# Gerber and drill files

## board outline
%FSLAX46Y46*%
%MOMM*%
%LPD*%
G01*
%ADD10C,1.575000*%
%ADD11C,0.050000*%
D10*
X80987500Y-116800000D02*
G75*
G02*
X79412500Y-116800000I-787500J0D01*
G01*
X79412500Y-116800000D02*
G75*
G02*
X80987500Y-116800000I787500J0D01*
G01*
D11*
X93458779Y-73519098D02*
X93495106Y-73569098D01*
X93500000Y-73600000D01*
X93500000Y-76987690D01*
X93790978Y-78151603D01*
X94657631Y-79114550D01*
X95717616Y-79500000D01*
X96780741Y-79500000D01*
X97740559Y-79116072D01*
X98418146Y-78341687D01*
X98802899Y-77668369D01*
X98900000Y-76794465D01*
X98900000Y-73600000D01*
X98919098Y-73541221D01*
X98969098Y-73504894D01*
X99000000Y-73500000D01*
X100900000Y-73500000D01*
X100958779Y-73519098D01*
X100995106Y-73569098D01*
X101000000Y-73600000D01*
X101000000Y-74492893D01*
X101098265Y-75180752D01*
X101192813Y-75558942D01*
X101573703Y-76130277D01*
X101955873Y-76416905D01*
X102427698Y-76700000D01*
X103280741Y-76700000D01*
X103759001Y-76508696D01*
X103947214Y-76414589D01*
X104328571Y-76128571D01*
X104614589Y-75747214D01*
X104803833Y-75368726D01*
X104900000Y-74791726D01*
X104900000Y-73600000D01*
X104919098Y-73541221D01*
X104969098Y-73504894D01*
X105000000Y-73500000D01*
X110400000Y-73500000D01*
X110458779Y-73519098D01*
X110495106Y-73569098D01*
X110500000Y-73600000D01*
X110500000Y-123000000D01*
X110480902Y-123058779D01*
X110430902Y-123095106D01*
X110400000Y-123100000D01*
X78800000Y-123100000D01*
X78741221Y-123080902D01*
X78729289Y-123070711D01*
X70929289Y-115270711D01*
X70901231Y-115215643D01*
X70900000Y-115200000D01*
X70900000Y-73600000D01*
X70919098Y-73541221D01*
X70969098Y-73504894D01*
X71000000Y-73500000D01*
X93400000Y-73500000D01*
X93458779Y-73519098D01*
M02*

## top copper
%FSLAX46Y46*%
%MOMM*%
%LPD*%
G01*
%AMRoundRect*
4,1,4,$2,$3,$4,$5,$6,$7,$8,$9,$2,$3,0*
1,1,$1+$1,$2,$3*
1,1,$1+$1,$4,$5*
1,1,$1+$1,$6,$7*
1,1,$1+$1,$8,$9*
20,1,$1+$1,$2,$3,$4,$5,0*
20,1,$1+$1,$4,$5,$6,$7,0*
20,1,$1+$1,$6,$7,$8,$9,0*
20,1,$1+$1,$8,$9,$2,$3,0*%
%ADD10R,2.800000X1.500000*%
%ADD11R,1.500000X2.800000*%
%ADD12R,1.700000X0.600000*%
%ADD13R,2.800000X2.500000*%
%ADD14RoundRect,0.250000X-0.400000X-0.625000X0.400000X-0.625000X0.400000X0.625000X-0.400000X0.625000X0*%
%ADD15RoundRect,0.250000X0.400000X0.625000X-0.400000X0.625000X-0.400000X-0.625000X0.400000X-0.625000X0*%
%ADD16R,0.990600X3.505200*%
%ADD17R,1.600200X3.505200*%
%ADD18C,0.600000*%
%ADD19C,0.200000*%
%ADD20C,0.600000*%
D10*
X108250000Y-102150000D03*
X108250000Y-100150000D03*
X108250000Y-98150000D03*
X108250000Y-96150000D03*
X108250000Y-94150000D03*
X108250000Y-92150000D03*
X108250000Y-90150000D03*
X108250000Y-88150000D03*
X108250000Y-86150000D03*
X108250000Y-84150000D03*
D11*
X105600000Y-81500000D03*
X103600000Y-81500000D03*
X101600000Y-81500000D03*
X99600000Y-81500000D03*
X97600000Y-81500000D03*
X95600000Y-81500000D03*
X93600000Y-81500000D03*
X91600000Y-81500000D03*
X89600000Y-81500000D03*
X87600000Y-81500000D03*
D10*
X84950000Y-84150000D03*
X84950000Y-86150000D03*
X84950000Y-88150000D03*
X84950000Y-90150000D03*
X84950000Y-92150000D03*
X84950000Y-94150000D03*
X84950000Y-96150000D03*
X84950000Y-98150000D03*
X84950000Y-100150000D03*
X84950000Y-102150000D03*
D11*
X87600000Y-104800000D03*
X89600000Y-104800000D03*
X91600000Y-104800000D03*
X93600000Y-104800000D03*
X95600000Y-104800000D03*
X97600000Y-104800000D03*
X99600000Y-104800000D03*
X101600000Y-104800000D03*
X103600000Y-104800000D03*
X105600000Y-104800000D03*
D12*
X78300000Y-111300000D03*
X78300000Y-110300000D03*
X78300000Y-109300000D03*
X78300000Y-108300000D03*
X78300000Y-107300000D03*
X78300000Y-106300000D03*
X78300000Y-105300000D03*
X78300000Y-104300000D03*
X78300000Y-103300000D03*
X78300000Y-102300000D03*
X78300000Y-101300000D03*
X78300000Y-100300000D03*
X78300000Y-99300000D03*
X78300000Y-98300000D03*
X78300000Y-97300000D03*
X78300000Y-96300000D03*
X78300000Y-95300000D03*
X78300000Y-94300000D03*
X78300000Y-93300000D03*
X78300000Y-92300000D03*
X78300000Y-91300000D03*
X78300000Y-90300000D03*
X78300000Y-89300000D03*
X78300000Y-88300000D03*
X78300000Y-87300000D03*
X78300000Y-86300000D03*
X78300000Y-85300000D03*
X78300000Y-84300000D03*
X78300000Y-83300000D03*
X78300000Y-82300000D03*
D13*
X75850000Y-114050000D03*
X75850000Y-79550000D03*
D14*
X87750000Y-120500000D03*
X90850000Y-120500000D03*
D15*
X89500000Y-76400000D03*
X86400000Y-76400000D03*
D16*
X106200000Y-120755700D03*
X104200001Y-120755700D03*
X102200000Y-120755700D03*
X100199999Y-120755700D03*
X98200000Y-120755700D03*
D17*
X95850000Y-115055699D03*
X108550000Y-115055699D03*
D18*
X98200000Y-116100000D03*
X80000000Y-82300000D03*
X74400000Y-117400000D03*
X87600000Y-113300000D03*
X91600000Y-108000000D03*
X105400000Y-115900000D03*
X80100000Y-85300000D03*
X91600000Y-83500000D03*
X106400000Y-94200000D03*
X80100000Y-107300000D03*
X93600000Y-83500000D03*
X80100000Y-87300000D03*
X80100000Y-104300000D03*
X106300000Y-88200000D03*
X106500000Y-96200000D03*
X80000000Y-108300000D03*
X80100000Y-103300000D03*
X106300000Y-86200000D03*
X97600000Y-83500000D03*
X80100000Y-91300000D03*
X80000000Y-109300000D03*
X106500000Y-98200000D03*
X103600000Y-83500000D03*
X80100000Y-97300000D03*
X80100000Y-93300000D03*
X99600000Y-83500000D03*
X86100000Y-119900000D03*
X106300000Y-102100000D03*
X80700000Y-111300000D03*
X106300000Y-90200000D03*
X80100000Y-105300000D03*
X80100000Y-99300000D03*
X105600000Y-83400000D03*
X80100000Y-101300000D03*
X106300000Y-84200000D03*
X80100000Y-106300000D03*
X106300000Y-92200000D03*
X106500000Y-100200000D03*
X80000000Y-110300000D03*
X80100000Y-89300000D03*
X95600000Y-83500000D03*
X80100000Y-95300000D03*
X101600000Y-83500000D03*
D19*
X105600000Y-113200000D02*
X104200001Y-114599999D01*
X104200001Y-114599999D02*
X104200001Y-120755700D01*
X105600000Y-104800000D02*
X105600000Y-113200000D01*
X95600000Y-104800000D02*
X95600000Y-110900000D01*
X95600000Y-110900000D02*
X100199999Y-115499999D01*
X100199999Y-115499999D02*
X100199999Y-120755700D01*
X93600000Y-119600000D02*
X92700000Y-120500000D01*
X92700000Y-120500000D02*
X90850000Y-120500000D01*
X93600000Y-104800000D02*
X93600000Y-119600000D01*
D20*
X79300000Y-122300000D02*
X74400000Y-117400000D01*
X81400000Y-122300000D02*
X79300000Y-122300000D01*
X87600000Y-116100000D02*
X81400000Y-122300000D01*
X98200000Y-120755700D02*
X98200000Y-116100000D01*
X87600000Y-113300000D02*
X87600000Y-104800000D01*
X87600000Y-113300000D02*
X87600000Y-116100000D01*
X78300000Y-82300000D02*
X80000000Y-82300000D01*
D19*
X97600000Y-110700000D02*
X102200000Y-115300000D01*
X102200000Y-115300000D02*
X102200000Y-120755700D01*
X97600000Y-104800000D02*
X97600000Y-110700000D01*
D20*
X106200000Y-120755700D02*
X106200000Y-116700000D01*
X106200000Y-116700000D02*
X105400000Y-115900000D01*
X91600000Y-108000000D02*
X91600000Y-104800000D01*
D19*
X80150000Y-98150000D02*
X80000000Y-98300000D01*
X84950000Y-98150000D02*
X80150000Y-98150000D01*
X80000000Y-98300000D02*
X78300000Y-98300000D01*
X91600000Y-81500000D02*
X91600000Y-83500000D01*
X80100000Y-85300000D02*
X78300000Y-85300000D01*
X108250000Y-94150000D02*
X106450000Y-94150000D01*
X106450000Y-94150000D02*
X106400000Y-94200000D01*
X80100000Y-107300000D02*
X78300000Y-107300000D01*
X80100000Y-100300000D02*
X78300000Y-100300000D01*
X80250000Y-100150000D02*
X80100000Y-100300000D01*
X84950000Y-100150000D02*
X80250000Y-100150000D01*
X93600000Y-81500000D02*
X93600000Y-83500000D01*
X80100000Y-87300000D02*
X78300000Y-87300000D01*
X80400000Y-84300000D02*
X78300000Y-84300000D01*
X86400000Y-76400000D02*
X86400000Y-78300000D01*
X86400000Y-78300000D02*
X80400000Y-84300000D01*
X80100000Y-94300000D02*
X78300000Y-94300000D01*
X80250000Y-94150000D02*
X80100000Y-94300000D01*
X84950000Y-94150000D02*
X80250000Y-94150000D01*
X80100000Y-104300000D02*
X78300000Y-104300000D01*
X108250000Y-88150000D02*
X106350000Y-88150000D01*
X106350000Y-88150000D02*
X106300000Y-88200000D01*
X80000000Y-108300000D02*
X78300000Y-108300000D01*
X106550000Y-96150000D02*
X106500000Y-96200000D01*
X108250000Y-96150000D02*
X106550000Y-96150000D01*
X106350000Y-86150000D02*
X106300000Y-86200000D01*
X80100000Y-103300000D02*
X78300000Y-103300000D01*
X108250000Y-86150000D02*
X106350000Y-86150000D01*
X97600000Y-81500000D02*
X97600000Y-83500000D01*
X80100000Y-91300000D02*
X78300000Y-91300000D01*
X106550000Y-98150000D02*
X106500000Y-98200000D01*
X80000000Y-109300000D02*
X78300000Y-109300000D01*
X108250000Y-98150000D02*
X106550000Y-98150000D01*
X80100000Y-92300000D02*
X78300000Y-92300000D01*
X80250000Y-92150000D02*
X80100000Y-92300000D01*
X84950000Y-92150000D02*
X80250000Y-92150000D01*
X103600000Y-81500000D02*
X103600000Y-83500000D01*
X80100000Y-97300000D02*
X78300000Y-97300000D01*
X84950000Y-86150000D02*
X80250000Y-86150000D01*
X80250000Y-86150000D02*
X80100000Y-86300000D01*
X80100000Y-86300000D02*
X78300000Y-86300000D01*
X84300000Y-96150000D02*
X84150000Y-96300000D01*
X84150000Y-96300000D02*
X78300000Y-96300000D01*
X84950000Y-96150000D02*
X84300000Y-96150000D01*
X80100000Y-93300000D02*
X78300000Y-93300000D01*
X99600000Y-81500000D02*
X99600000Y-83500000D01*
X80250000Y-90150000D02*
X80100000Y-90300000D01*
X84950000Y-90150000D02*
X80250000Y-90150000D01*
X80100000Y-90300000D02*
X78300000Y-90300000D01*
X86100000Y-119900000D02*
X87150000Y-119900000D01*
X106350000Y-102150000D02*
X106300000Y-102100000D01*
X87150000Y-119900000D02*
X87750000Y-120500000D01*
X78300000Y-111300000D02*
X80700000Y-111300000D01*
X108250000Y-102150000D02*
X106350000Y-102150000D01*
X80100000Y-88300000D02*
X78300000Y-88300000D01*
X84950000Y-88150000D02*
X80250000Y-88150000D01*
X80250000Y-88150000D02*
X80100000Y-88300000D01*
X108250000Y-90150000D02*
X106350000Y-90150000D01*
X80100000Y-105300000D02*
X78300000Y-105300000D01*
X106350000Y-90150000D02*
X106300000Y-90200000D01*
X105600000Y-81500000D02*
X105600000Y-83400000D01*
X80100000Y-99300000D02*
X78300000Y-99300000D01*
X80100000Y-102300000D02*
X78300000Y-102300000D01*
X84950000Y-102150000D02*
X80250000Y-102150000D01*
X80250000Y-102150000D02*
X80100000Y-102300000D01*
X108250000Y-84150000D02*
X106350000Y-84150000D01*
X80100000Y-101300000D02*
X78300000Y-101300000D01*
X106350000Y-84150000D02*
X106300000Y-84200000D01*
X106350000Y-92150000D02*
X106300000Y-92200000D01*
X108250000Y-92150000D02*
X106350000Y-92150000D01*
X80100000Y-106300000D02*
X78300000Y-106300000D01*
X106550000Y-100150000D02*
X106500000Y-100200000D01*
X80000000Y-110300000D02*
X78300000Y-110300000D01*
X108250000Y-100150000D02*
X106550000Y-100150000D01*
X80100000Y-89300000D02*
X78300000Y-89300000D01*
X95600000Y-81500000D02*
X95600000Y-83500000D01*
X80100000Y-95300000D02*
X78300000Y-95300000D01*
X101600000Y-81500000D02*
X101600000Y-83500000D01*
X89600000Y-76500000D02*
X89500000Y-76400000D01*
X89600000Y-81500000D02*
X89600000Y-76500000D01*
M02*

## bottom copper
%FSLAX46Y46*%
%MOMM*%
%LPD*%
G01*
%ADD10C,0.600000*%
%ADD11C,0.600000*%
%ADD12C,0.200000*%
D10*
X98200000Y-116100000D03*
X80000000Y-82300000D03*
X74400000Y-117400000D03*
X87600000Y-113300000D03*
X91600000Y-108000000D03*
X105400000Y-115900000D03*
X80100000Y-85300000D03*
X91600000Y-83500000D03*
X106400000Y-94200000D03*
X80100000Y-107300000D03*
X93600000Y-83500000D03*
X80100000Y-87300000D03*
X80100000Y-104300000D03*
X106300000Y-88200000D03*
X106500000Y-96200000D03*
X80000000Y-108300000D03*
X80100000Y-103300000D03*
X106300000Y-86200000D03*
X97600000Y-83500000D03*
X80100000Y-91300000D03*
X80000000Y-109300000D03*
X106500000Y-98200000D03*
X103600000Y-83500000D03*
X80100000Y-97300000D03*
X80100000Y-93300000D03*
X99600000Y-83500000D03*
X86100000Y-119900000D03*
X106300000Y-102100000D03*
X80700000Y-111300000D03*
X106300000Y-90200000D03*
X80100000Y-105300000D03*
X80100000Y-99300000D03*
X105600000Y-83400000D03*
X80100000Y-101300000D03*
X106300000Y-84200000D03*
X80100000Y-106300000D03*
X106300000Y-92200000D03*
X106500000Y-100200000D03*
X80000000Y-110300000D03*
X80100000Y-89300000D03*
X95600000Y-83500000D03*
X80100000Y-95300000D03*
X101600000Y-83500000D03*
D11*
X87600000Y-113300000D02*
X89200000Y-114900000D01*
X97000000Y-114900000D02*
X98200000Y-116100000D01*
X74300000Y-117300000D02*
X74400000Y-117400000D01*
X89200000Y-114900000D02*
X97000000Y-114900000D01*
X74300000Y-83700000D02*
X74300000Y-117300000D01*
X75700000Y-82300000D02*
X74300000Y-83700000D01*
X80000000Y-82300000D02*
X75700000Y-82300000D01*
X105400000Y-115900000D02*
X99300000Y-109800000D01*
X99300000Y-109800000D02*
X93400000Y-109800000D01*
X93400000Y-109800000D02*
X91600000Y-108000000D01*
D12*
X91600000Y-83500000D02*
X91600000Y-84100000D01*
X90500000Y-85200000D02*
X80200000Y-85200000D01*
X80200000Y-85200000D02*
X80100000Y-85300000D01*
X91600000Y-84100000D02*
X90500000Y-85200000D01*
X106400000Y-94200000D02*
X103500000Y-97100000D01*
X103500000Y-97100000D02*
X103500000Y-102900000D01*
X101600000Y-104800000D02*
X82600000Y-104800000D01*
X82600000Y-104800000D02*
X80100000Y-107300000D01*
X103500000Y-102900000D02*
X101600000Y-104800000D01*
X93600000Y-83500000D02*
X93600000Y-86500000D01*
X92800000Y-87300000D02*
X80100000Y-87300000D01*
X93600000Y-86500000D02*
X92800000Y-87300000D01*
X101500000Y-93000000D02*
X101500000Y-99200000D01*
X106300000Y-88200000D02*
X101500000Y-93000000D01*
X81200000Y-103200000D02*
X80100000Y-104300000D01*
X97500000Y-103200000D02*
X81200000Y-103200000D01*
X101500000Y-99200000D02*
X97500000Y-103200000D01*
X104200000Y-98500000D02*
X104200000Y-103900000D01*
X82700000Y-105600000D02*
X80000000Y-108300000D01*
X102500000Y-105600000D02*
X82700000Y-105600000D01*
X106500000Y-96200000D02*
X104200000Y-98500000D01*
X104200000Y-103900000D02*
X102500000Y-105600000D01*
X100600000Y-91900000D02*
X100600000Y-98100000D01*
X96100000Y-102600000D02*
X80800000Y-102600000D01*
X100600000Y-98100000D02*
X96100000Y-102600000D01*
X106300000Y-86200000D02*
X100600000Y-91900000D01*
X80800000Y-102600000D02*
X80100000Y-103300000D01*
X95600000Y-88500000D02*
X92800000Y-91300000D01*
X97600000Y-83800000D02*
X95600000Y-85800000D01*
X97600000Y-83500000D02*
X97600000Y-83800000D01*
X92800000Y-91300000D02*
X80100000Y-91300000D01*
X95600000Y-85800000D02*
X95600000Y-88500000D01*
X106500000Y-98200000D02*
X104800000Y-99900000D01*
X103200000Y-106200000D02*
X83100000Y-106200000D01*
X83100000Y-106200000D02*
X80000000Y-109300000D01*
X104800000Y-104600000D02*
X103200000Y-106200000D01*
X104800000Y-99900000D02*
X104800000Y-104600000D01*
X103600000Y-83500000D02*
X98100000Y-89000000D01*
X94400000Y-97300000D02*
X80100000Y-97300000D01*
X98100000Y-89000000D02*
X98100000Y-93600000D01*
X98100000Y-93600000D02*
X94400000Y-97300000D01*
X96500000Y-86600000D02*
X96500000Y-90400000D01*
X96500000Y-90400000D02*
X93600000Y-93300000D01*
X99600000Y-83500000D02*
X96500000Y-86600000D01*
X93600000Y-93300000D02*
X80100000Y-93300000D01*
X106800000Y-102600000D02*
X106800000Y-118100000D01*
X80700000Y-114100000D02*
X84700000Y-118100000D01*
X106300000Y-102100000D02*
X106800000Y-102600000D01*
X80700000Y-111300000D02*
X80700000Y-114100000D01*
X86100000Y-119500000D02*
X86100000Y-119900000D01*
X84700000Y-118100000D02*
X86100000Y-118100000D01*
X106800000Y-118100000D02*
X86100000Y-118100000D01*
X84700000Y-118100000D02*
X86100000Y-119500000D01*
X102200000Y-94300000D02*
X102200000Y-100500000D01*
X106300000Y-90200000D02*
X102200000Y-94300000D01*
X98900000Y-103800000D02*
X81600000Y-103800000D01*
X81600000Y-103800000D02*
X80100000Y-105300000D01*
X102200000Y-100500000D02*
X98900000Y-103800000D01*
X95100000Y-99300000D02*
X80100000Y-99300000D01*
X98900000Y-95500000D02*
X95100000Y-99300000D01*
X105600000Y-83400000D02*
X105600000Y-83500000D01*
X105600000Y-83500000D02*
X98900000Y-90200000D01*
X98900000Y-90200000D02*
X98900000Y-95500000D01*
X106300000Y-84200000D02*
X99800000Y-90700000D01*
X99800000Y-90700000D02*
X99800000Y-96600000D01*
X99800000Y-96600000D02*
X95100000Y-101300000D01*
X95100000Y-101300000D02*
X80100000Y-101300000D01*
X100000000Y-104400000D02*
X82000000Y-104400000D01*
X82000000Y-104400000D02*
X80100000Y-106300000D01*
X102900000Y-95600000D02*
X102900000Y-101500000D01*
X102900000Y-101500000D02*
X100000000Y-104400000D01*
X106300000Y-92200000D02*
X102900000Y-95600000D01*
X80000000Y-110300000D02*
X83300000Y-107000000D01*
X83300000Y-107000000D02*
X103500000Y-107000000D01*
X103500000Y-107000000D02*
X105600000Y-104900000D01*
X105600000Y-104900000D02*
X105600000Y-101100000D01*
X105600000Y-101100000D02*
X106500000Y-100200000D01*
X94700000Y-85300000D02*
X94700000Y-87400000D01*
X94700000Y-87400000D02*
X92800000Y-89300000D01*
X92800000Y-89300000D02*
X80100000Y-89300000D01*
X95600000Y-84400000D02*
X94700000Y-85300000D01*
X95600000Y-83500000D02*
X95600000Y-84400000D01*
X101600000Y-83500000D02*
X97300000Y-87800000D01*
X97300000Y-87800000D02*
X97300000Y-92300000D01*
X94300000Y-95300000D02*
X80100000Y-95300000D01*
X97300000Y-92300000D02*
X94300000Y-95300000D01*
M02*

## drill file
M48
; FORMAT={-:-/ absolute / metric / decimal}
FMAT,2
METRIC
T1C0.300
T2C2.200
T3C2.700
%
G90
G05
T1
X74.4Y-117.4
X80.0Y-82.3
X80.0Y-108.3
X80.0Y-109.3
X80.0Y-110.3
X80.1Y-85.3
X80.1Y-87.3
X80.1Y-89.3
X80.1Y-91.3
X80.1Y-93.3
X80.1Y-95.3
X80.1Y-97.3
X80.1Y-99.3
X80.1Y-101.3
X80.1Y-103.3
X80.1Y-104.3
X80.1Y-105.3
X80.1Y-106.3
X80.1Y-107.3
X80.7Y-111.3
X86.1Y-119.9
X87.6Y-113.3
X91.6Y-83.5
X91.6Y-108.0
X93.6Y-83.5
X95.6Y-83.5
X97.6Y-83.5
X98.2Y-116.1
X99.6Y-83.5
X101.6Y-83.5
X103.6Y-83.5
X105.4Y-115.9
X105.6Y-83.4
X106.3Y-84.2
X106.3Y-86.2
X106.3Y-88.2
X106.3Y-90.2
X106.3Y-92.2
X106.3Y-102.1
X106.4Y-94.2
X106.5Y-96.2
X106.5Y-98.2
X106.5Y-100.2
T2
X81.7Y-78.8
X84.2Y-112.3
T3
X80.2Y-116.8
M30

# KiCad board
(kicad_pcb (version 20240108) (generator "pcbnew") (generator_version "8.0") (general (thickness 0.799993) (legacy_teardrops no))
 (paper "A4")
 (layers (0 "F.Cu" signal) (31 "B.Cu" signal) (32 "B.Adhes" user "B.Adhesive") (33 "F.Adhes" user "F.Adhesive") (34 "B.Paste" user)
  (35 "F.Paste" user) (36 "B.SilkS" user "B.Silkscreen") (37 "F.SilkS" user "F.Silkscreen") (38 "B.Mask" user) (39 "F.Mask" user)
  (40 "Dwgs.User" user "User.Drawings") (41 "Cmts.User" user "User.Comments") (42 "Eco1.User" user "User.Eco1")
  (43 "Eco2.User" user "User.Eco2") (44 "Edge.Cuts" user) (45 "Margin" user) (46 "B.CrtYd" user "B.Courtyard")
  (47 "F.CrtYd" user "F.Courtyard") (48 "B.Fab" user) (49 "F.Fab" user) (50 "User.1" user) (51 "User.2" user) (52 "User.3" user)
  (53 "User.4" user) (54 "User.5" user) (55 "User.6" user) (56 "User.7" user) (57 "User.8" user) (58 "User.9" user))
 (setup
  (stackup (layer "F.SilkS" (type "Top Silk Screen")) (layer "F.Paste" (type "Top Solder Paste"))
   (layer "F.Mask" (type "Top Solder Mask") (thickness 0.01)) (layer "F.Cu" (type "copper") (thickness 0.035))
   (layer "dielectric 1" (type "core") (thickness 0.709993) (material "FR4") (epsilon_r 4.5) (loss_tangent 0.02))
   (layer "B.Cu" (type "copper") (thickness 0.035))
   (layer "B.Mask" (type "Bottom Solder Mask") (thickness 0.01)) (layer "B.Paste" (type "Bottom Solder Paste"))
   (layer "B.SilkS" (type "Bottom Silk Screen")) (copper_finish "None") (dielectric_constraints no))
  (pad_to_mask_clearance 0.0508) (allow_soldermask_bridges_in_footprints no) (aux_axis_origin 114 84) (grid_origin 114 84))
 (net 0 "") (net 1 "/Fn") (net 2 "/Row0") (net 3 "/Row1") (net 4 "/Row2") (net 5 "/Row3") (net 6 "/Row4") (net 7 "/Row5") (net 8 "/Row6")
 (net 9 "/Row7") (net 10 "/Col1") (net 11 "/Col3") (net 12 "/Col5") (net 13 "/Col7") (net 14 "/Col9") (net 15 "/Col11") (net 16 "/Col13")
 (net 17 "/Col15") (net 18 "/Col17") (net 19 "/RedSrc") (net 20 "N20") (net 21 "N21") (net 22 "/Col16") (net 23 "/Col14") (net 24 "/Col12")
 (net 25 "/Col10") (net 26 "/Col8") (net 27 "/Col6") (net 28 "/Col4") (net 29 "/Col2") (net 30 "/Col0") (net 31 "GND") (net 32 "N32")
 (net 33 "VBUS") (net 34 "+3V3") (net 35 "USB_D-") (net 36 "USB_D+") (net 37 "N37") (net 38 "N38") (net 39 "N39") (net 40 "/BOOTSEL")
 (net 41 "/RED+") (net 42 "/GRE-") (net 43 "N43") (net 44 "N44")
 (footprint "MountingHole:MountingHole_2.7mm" (layer "F.Cu") (at 80.2 116.8)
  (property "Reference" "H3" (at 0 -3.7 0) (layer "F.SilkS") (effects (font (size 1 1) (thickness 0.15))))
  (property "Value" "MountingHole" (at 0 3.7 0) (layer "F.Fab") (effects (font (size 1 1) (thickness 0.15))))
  (pad "" np_thru_hole circle (at 0 0) (size 2.7 2.7) (drill 2.7) (layers "*.Cu" "*.Mask")))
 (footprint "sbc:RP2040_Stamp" (layer "F.Cu") (at 96.6 93.15 180)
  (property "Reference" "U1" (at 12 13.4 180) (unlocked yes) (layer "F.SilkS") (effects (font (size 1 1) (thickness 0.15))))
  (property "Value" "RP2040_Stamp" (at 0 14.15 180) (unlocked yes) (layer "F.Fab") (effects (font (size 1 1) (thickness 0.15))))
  (pad "1" smd rect (at -11.65 -9 180) (size 2.8 1.5) (layers "F.Cu" "F.Paste" "F.Mask") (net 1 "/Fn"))
  (pad "2" smd rect (at -11.65 -7 180) (size 2.8 1.5) (layers "F.Cu" "F.Paste" "F.Mask") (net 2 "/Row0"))
  (pad "3" smd rect (at -11.65 -5 180) (size 2.8 1.5) (layers "F.Cu" "F.Paste" "F.Mask") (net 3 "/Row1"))
  (pad "4" smd rect (at -11.65 -3 180) (size 2.8 1.5) (layers "F.Cu" "F.Paste" "F.Mask") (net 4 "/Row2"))
  (pad "5" smd rect (at -11.65 -1 180) (size 2.8 1.5) (layers "F.Cu" "F.Paste" "F.Mask") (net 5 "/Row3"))
  (pad "6" smd rect (at -11.65 1 180) (size 2.8 1.5) (layers "F.Cu" "F.Paste" "F.Mask") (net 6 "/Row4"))
  (pad "7" smd rect (at -11.65 3 180) (size 2.8 1.5) (layers "F.Cu" "F.Paste" "F.Mask") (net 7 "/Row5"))
  (pad "8" smd rect (at -11.65 5 180) (size 2.8 1.5) (layers "F.Cu" "F.Paste" "F.Mask") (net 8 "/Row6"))
  (pad "9" smd rect (at -11.65 7 180) (size 2.8 1.5) (layers "F.Cu" "F.Paste" "F.Mask") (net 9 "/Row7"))
  (pad "10" smd rect (at -11.65 9 180) (size 2.8 1.5) (layers "F.Cu" "F.Paste" "F.Mask") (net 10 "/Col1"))
  (pad "11" smd rect (at -9 11.65 90) (size 2.8 1.5) (layers "F.Cu" "F.Paste" "F.Mask") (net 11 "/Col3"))
  (pad "12" smd rect (at -7 11.65 90) (size 2.8 1.5) (layers "F.Cu" "F.Paste" "F.Mask") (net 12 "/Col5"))
  (pad "13" smd rect (at -5 11.65 90) (size 2.8 1.5) (layers "F.Cu" "F.Paste" "F.Mask") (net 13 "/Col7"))
  (pad "14" smd rect (at -3 11.65 90) (size 2.8 1.5) (layers "F.Cu" "F.Paste" "F.Mask") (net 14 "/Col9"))
  (pad "15" smd rect (at -1 11.65 90) (size 2.8 1.5) (layers "F.Cu" "F.Paste" "F.Mask") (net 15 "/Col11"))
  (pad "16" smd rect (at 1 11.65 90) (size 2.8 1.5) (layers "F.Cu" "F.Paste" "F.Mask") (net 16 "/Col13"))
  (pad "17" smd rect (at 3 11.65 90) (size 2.8 1.5) (layers "F.Cu" "F.Paste" "F.Mask") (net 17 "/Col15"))
  (pad "18" smd rect (at 5 11.65 90) (size 2.8 1.5) (layers "F.Cu" "F.Paste" "F.Mask") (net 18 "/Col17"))
  (pad "19" smd rect (at 7 11.65 90) (size 2.8 1.5) (layers "F.Cu" "F.Paste" "F.Mask") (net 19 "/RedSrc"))
  (pad "20" smd rect (at 9 11.65 90) (size 2.8 1.5) (layers "F.Cu" "F.Paste" "F.Mask") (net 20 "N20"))
  (pad "21" smd rect (at 11.65 9 180) (size 2.8 1.5) (layers "F.Cu" "F.Paste" "F.Mask") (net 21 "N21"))
  (pad "22" smd rect (at 11.65 7 180) (size 2.8 1.5) (layers "F.Cu" "F.Paste" "F.Mask") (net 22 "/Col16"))
  (pad "23" smd rect (at 11.65 5 180) (size 2.8 1.5) (layers "F.Cu" "F.Paste" "F.Mask") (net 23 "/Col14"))
  (pad "24" smd rect (at 11.65 3 180) (size 2.8 1.5) (layers "F.Cu" "F.Paste" "F.Mask") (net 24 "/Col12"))
  (pad "25" smd rect (at 11.65 1 180) (size 2.8 1.5) (layers "F.Cu" "F.Paste" "F.Mask") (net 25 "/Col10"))
  (pad "26" smd rect (at 11.65 -1 180) (size 2.8 1.5) (layers "F.Cu" "F.Paste" "F.Mask") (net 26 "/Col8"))
  (pad "27" smd rect (at 11.65 -3 180) (size 2.8 1.5) (layers "F.Cu" "F.Paste" "F.Mask") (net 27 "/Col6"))
  (pad "28" smd rect (at 11.65 -5 180) (size 2.8 1.5) (layers "F.Cu" "F.Paste" "F.Mask") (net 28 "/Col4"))
  (pad "29" smd rect (at 11.65 -7 180) (size 2.8 1.5) (layers "F.Cu" "F.Paste" "F.Mask") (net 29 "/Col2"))
  (pad "30" smd rect (at 11.65 -9 180) (size 2.8 1.5) (layers "F.Cu" "F.Paste" "F.Mask") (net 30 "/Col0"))
  (pad "31" smd rect (at 9 -11.65 90) (size 2.8 1.5) (layers "F.Cu" "F.Paste" "F.Mask") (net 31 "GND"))
  (pad "32" smd rect (at 7 -11.65 90) (size 2.8 1.5) (layers "F.Cu" "F.Paste" "F.Mask") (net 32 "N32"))
  (pad "33" smd rect (at 5 -11.65 90) (size 2.8 1.5) (layers "F.Cu" "F.Paste" "F.Mask") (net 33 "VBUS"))
  (pad "34" smd rect (at 3 -11.65 90) (size 2.8 1.5) (layers "F.Cu" "F.Paste" "F.Mask") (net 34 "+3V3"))
  (pad "35" smd rect (at 1 -11.65 90) (size 2.8 1.5) (layers "F.Cu" "F.Paste" "F.Mask") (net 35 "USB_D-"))
  (pad "36" smd rect (at -1 -11.65 90) (size 2.8 1.5) (layers "F.Cu" "F.Paste" "F.Mask") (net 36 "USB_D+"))
  (pad "37" smd rect (at -3 -11.65 90) (size 2.8 1.5) (layers "F.Cu" "F.Paste" "F.Mask") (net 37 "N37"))
  (pad "38" smd rect (at -5 -11.65 90) (size 2.8 1.5) (layers "F.Cu" "F.Paste" "F.Mask") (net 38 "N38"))
  (pad "39" smd rect (at -7 -11.65 90) (size 2.8 1.5) (layers "F.Cu" "F.Paste" "F.Mask") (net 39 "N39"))
  (pad "40" smd rect (at -9 -11.65 90) (size 2.8 1.5) (layers "F.Cu" "F.Paste" "F.Mask") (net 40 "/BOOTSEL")))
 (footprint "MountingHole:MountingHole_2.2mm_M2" (layer "F.Cu") (at 81.7 78.8)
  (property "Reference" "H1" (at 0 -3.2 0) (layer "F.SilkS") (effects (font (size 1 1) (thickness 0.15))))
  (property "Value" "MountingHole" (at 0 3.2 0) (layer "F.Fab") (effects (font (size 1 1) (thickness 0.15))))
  (pad "" np_thru_hole circle (at 0 0) (size 2.2 2.2) (drill 2.2) (layers "*.Cu" "*.Mask")))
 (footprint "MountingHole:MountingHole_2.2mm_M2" (layer "F.Cu") (at 84.2 112.3)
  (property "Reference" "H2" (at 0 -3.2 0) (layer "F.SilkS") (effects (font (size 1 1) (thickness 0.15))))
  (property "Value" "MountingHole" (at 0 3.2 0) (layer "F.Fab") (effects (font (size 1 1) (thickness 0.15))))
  (pad "" np_thru_hole circle (at 0 0) (size 2.2 2.2) (drill 2.2) (layers "*.Cu" "*.Mask")))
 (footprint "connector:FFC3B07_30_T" (layer "F.Cu") (at 75.85 96.8 -90)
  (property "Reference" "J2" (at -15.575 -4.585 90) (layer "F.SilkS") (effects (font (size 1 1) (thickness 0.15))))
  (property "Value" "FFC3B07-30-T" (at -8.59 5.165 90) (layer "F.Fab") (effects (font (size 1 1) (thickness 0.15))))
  (pad "1" smd rect (at 14.5 -2.45 270) (size 0.6 1.7) (layers "F.Cu" "F.Paste" "F.Mask") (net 1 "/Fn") (solder_mask_margin 0.102))
  (pad "2" smd rect (at 13.5 -2.45 270) (size 0.6 1.7) (layers "F.Cu" "F.Paste" "F.Mask") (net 2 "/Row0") (solder_mask_margin 0.102))
  (pad "3" smd rect (at 12.5 -2.45 270) (size 0.6 1.7) (layers "F.Cu" "F.Paste" "F.Mask") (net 3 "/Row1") (solder_mask_margin 0.102))
  (pad "4" smd rect (at 11.5 -2.45 270) (size 0.6 1.7) (layers "F.Cu" "F.Paste" "F.Mask") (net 4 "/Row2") (solder_mask_margin 0.102))
  (pad "5" smd rect (at 10.5 -2.45 270) (size 0.6 1.7) (layers "F.Cu" "F.Paste" "F.Mask") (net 5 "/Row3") (solder_mask_margin 0.102))
  (pad "6" smd rect (at 9.5 -2.45 270) (size 0.6 1.7) (layers "F.Cu" "F.Paste" "F.Mask") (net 6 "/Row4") (solder_mask_margin 0.102))
  (pad "7" smd rect (at 8.5 -2.45 270) (size 0.6 1.7) (layers "F.Cu" "F.Paste" "F.Mask") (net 7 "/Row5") (solder_mask_margin 0.102))
  (pad "8" smd rect (at 7.5 -2.45 270) (size 0.6 1.7) (layers "F.Cu" "F.Paste" "F.Mask") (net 8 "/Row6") (solder_mask_margin 0.102))
  (pad "9" smd rect (at 6.5 -2.45 270) (size 0.6 1.7) (layers "F.Cu" "F.Paste" "F.Mask") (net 9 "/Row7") (solder_mask_margin 0.102))
  (pad "10" smd rect (at 5.5 -2.45 270) (size 0.6 1.7) (layers "F.Cu" "F.Paste" "F.Mask") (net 30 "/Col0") (solder_mask_margin 0.102))
  (pad "11" smd rect (at 4.5 -2.45 270) (size 0.6 1.7) (layers "F.Cu" "F.Paste" "F.Mask") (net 10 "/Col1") (solder_mask_margin 0.102))
  (pad "12" smd rect (at 3.5 -2.45 270) (size 0.6 1.7) (layers "F.Cu" "F.Paste" "F.Mask") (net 29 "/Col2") (solder_mask_margin 0.102))
  (pad "13" smd rect (at 2.5 -2.45 270) (size 0.6 1.7) (layers "F.Cu" "F.Paste" "F.Mask") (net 11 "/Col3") (solder_mask_margin 0.102))
  (pad "14" smd rect (at 1.5 -2.45 270) (size 0.6 1.7) (layers "F.Cu" "F.Paste" "F.Mask") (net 28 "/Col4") (solder_mask_margin 0.102))
  (pad "15" smd rect (at 0.5 -2.45 270) (size 0.6 1.7) (layers "F.Cu" "F.Paste" "F.Mask") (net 12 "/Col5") (solder_mask_margin 0.102))
  (pad "16" smd rect (at -0.5 -2.45 270) (size 0.6 1.7) (layers "F.Cu" "F.Paste" "F.Mask") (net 27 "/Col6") (solder_mask_margin 0.102))
  (pad "17" smd rect (at -1.5 -2.45 270) (size 0.6 1.7) (layers "F.Cu" "F.Paste" "F.Mask") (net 13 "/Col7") (solder_mask_margin 0.102))
  (pad "18" smd rect (at -2.5 -2.45 270) (size 0.6 1.7) (layers "F.Cu" "F.Paste" "F.Mask") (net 26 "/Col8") (solder_mask_margin 0.102))
  (pad "19" smd rect (at -3.5 -2.45 270) (size 0.6 1.7) (layers "F.Cu" "F.Paste" "F.Mask") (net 14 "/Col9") (solder_mask_margin 0.102))
  (pad "20" smd rect (at -4.5 -2.45 270) (size 0.6 1.7) (layers "F.Cu" "F.Paste" "F.Mask") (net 25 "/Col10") (solder_mask_margin 0.102))
  (pad "21" smd rect (at -5.5 -2.45 270) (size 0.6 1.7) (layers "F.Cu" "F.Paste" "F.Mask") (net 15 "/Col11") (solder_mask_margin 0.102))
  (pad "22" smd rect (at -6.5 -2.45 270) (size 0.6 1.7) (layers "F.Cu" "F.Paste" "F.Mask") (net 24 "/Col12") (solder_mask_margin 0.102))
  (pad "23" smd rect (at -7.5 -2.45 270) (size 0.6 1.7) (layers "F.Cu" "F.Paste" "F.Mask") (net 16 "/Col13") (solder_mask_margin 0.102))
  (pad "24" smd rect (at -8.5 -2.45 270) (size 0.6 1.7) (layers "F.Cu" "F.Paste" "F.Mask") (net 23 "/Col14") (solder_mask_margin 0.102))
  (pad "25" smd rect (at -9.5 -2.45 270) (size 0.6 1.7) (layers "F.Cu" "F.Paste" "F.Mask") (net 17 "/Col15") (solder_mask_margin 0.102))
  (pad "26" smd rect (at -10.5 -2.45 270) (size 0.6 1.7) (layers "F.Cu" "F.Paste" "F.Mask") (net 22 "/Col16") (solder_mask_margin 0.102))
  (pad "27" smd rect (at -11.5 -2.45 270) (size 0.6 1.7) (layers "F.Cu" "F.Paste" "F.Mask") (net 18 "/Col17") (solder_mask_margin 0.102))
  (pad "28" smd rect (at -12.5 -2.45 270) (size 0.6 1.7) (layers "F.Cu" "F.Paste" "F.Mask") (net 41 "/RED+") (solder_mask_margin 0.102))
  (pad "29" smd rect (at -13.5 -2.45 270) (size 0.6 1.7) (layers "F.Cu" "F.Paste" "F.Mask") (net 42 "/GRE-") (solder_mask_margin 0.102))
  (pad "30" smd rect (at -14.5 -2.45 270) (size 0.6 1.7) (layers "F.Cu" "F.Paste" "F.Mask") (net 31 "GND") (solder_mask_margin 0.102))
  (pad "S1" smd rect (at 17.25 0 270) (size 2.5 2.8) (layers "F.Cu" "F.Paste" "F.Mask") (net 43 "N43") (solder_mask_margin 0.102))
  (pad "S2" smd rect (at -17.25 0 270) (size 2.5 2.8) (layers "F.Cu" "F.Paste" "F.Mask") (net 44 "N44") (solder_mask_margin 0.102)))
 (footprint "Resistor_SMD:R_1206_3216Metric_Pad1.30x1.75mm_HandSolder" (layer "F.Cu") (at 89.3 120.5)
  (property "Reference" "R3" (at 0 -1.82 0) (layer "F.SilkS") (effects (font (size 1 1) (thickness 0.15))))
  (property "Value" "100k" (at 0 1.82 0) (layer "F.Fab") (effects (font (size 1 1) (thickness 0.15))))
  (pad "1" smd roundrect (at -1.55 0) (size 1.3 1.75) (layers "F.Cu" "F.Paste" "F.Mask") (roundrect_rratio 0.192308) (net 1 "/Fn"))
  (pad "2" smd roundrect (at 1.55 0) (size 1.3 1.75) (layers "F.Cu" "F.Paste" "F.Mask") (roundrect_rratio 0.192308) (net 34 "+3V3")))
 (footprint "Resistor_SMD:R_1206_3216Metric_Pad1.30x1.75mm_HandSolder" (layer "F.Cu") (at 87.95 76.4 180)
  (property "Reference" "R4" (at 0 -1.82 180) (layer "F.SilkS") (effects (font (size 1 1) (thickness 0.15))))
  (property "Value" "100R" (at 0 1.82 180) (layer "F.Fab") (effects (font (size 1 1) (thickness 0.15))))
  (pad "1" smd roundrect (at -1.55 0 180) (size 1.3 1.75) (layers "F.Cu" "F.Paste" "F.Mask") (roundrect_rratio 0.192308) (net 19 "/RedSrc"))
  (pad "2" smd roundrect (at 1.55 0 180) (size 1.3 1.75) (layers "F.Cu" "F.Paste" "F.Mask") (roundrect_rratio 0.192308) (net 41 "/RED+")))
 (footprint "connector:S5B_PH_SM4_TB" (layer "F.Cu") (at 102.2 117.3)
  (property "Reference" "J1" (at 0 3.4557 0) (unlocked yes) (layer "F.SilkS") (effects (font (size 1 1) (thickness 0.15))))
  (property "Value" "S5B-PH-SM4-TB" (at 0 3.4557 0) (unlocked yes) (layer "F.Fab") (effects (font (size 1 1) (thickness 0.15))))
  (pad "1" smd rect (at 4 3.4557) (size 0.9906 3.5052) (layers "F.Cu" "F.Paste" "F.Mask") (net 33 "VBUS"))
  (pad "2" smd rect (at 2.000001 3.4557) (size 0.9906 3.5052) (layers "F.Cu" "F.Paste" "F.Mask") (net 40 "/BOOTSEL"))
  (pad "3" smd rect (at 0 3.4557) (size 0.9906 3.5052) (layers "F.Cu" "F.Paste" "F.Mask") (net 36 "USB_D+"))
  (pad "4" smd rect (at -2.000001 3.4557) (size 0.9906 3.5052) (layers "F.Cu" "F.Paste" "F.Mask") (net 35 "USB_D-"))
  (pad "5" smd rect (at -4 3.4557) (size 0.9906 3.5052) (layers "F.Cu" "F.Paste" "F.Mask") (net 31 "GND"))
  (pad "6" smd rect (at -6.35 -2.244301) (size 1.6002 3.5052) (layers "F.Cu" "F.Paste" "F.Mask"))
  (pad "7" smd rect (at 6.35 -2.244301) (size 1.6002 3.5052) (layers "F.Cu" "F.Paste" "F.Mask")))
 (gr_circle (center 80.2 116.8) (end 81.75 116.8) (stroke (width 0.05) (type solid)) (fill solid) (layer "Edge.Cuts"))
 (gr_poly
  (pts (xy 93.458779 73.519098) (xy 93.495106 73.569098) (xy 93.5 73.6) (xy 93.5 76.98769) (xy 93.790978 78.151603) (xy 94.657631 79.11455)
   (xy 95.717616 79.5) (xy 96.780741 79.5) (xy 97.740559 79.116072) (xy 98.418146 78.341687) (xy 98.802899 77.668369) (xy 98.9 76.794465)
   (xy 98.9 73.6) (xy 98.919098 73.541221) (xy 98.969098 73.504894) (xy 99 73.5) (xy 100.9 73.5) (xy 100.958779 73.519098)
   (xy 100.995106 73.569098) (xy 101 73.6) (xy 101 74.492893) (xy 101.098265 75.180752) (xy 101.192813 75.558942) (xy 101.573703 76.130277)
   (xy 101.955873 76.416905) (xy 102.427698 76.7) (xy 103.280741 76.7) (xy 103.759001 76.508696) (xy 103.947214 76.414589)
   (xy 104.328571 76.128571) (xy 104.614589 75.747214) (xy 104.803833 75.368726) (xy 104.9 74.791726) (xy 104.9 73.6)
   (xy 104.919098 73.541221) (xy 104.969098 73.504894) (xy 105 73.5) (xy 110.4 73.5) (xy 110.458779 73.519098) (xy 110.495106 73.569098)
   (xy 110.5 73.6) (xy 110.5 123) (xy 110.480902 123.058779) (xy 110.430902 123.095106) (xy 110.4 123.1) (xy 78.8 123.1)
   (xy 78.741221 123.080902) (xy 78.729289 123.070711) (xy 70.929289 115.270711) (xy 70.901231 115.215643) (xy 70.9 115.2) (xy 70.9 73.6)
   (xy 70.919098 73.541221) (xy 70.969098 73.504894) (xy 71 73.5) (xy 93.4 73.5))
  (stroke (width 0.05) (type solid)) (fill none) (layer "Edge.Cuts"))
 (segment (start 105.6 113.2) (end 104.200001 114.599999) (width 0.2) (layer "F.Cu") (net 40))
 (segment (start 104.200001 114.599999) (end 104.200001 120.7557) (width 0.2) (layer "F.Cu") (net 40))
 (segment (start 105.6 104.8) (end 105.6 113.2) (width 0.2) (layer "F.Cu") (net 40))
 (segment (start 95.6 104.8) (end 95.6 110.9) (width 0.2) (layer "F.Cu") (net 35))
 (segment (start 95.6 110.9) (end 100.199999 115.499999) (width 0.2) (layer "F.Cu") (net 35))
 (segment (start 100.199999 115.499999) (end 100.199999 120.7557) (width 0.2) (layer "F.Cu") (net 35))
 (segment (start 93.6 119.6) (end 92.7 120.5) (width 0.2) (layer "F.Cu") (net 34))
 (segment (start 92.7 120.5) (end 90.85 120.5) (width 0.2) (layer "F.Cu") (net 34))
 (segment (start 93.6 104.8) (end 93.6 119.6) (width 0.2) (layer "F.Cu") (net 34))
 (segment (start 79.3 122.3) (end 74.4 117.4) (width 0.6) (layer "F.Cu") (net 31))
 (segment (start 81.4 122.3) (end 79.3 122.3) (width 0.6) (layer "F.Cu") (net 31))
 (segment (start 87.6 116.1) (end 81.4 122.3) (width 0.6) (layer "F.Cu") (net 31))
 (segment (start 98.2 120.7557) (end 98.2 116.1) (width 0.6) (layer "F.Cu") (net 31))
 (segment (start 87.6 113.3) (end 87.6 104.8) (width 0.6) (layer "F.Cu") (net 31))
 (segment (start 87.6 113.3) (end 87.6 116.1) (width 0.6) (layer "F.Cu") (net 31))
 (segment (start 78.3 82.3) (end 80 82.3) (width 0.6) (layer "F.Cu") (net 31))
 (via (at 98.2 116.1) (size 0.6) (drill 0.3) (layers "F.Cu" "B.Cu") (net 31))
 (via (at 80 82.3) (size 0.6) (drill 0.3) (layers "F.Cu" "B.Cu") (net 31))
 (via (at 74.4 117.4) (size 0.6) (drill 0.3) (layers "F.Cu" "B.Cu") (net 31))
 (via (at 87.6 113.3) (size 0.6) (drill 0.3) (layers "F.Cu" "B.Cu") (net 31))
 (segment (start 87.6 113.3) (end 89.2 114.9) (width 0.6) (layer "B.Cu") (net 31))
 (segment (start 97 114.9) (end 98.2 116.1) (width 0.6) (layer "B.Cu") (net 31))
 (segment (start 74.3 117.3) (end 74.4 117.4) (width 0.6) (layer "B.Cu") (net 31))
 (segment (start 89.2 114.9) (end 97 114.9) (width 0.6) (layer "B.Cu") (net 31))
 (segment (start 74.3 83.7) (end 74.3 117.3) (width 0.6) (layer "B.Cu") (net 31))
 (segment (start 75.7 82.3) (end 74.3 83.7) (width 0.6) (layer "B.Cu") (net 31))
 (segment (start 80 82.3) (end 75.7 82.3) (width 0.6) (layer "B.Cu") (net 31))
 (segment (start 97.6 110.7) (end 102.2 115.3) (width 0.2) (layer "F.Cu") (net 36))
 (segment (start 102.2 115.3) (end 102.2 120.7557) (width 0.2) (layer "F.Cu") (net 36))
 (segment (start 97.6 104.8) (end 97.6 110.7) (width 0.2) (layer "F.Cu") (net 36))
 (segment (start 106.2 120.7557) (end 106.2 116.7) (width 0.6) (layer "F.Cu") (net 33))
 (segment (start 106.2 116.7) (end 105.4 115.9) (width 0.6) (layer "F.Cu") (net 33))
 (segment (start 91.6 108) (end 91.6 104.8) (width 0.6) (layer "F.Cu") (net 33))
 (via (at 91.6 108) (size 0.6) (drill 0.3) (layers "F.Cu" "B.Cu") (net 33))
 (via (at 105.4 115.9) (size 0.6) (drill 0.3) (layers "F.Cu" "B.Cu") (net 33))
 (segment (start 105.4 115.9) (end 99.3 109.8) (width 0.6) (layer "B.Cu") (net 33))
 (segment (start 99.3 109.8) (end 93.4 109.8) (width 0.6) (layer "B.Cu") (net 33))
 (segment (start 93.4 109.8) (end 91.6 108) (width 0.6) (layer "B.Cu") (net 33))
 (segment (start 80.15 98.15) (end 80 98.3) (width 0.2) (layer "F.Cu") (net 28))
 (segment (start 84.95 98.15) (end 80.15 98.15) (width 0.2) (layer "F.Cu") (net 28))
 (segment (start 80 98.3) (end 78.3 98.3) (width 0.2) (layer "F.Cu") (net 28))
 (segment (start 91.6 81.5) (end 91.6 83.5) (width 0.2) (layer "F.Cu") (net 18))
 (segment (start 80.1 85.3) (end 78.3 85.3) (width 0.2) (layer "F.Cu") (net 18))
 (via (at 80.1 85.3) (size 0.6) (drill 0.3) (layers "F.Cu" "B.Cu") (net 18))
 (via (at 91.6 83.5) (size 0.6) (drill 0.3) (layers "F.Cu" "B.Cu") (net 18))
 (segment (start 91.6 83.5) (end 91.6 84.1) (width 0.2) (layer "B.Cu") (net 18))
 (segment (start 90.5 85.2) (end 80.2 85.2) (width 0.2) (layer "B.Cu") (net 18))
 (segment (start 80.2 85.2) (end 80.1 85.3) (width 0.2) (layer "B.Cu") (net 18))
 (segment (start 91.6 84.1) (end 90.5 85.2) (width 0.2) (layer "B.Cu") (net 18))
 (segment (start 108.25 94.15) (end 106.45 94.15) (width 0.2) (layer "F.Cu") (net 5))
 (segment (start 106.45 94.15) (end 106.4 94.2) (width 0.2) (layer "F.Cu") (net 5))
 (segment (start 80.1 107.3) (end 78.3 107.3) (width 0.2) (layer "F.Cu") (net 5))
 (via (at 106.4 94.2) (size 0.6) (drill 0.3) (layers "F.Cu" "B.Cu") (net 5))
 (via (at 80.1 107.3) (size 0.6) (drill 0.3) (layers "F.Cu" "B.Cu") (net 5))
 (segment (start 106.4 94.2) (end 103.5 97.1) (width 0.2) (layer "B.Cu") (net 5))
 (segment (start 103.5 97.1) (end 103.5 102.9) (width 0.2) (layer "B.Cu") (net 5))
 (segment (start 101.6 104.8) (end 82.6 104.8) (width 0.2) (layer "B.Cu") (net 5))
 (segment (start 82.6 104.8) (end 80.1 107.3) (width 0.2) (layer "B.Cu") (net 5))
 (segment (start 103.5 102.9) (end 101.6 104.8) (width 0.2) (layer "B.Cu") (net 5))
 (segment (start 80.1 100.3) (end 78.3 100.3) (width 0.2) (layer "F.Cu") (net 29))
 (segment (start 80.25 100.15) (end 80.1 100.3) (width 0.2) (layer "F.Cu") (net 29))
 (segment (start 84.95 100.15) (end 80.25 100.15) (width 0.2) (layer "F.Cu") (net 29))
 (segment (start 93.6 81.5) (end 93.6 83.5) (width 0.2) (layer "F.Cu") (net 17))
 (segment (start 80.1 87.3) (end 78.3 87.3) (width 0.2) (layer "F.Cu") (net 17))
 (via (at 93.6 83.5) (size 0.6) (drill 0.3) (layers "F.Cu" "B.Cu") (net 17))
 (via (at 80.1 87.3) (size 0.6) (drill 0.3) (layers "F.Cu" "B.Cu") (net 17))
 (segment (start 93.6 83.5) (end 93.6 86.5) (width 0.2) (layer "B.Cu") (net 17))
 (segment (start 92.8 87.3) (end 80.1 87.3) (width 0.2) (layer "B.Cu") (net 17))
 (segment (start 93.6 86.5) (end 92.8 87.3) (width 0.2) (layer "B.Cu") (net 17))
 (segment (start 80.4 84.3) (end 78.3 84.3) (width 0.2) (layer "F.Cu") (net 41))
 (segment (start 86.4 76.4) (end 86.4 78.3) (width 0.2) (layer "F.Cu") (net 41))
 (segment (start 86.4 78.3) (end 80.4 84.3) (width 0.2) (layer "F.Cu") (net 41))
 (segment (start 80.1 94.3) (end 78.3 94.3) (width 0.2) (layer "F.Cu") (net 26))
 (segment (start 80.25 94.15) (end 80.1 94.3) (width 0.2) (layer "F.Cu") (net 26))
 (segment (start 84.95 94.15) (end 80.25 94.15) (width 0.2) (layer "F.Cu") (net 26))
 (segment (start 80.1 104.3) (end 78.3 104.3) (width 0.2) (layer "F.Cu") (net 8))
 (segment (start 108.25 88.15) (end 106.35 88.15) (width 0.2) (layer "F.Cu") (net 8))
 (segment (start 106.35 88.15) (end 106.3 88.2) (width 0.2) (layer "F.Cu") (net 8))
 (via (at 80.1 104.3) (size 0.6) (drill 0.3) (layers "F.Cu" "B.Cu") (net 8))
 (via (at 106.3 88.2) (size 0.6) (drill 0.3) (layers "F.Cu" "B.Cu") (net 8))
 (segment (start 101.5 93) (end 101.5 99.2) (width 0.2) (layer "B.Cu") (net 8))
 (segment (start 106.3 88.2) (end 101.5 93) (width 0.2) (layer "B.Cu") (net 8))
 (segment (start 81.2 103.2) (end 80.1 104.3) (width 0.2) (layer "B.Cu") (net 8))
 (segment (start 97.5 103.2) (end 81.2 103.2) (width 0.2) (layer "B.Cu") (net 8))
 (segment (start 101.5 99.2) (end 97.5 103.2) (width 0.2) (layer "B.Cu") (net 8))
 (segment (start 80 108.3) (end 78.3 108.3) (width 0.2) (layer "F.Cu") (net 4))
 (segment (start 106.55 96.15) (end 106.5 96.2) (width 0.2) (layer "F.Cu") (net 4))
 (segment (start 108.25 96.15) (end 106.55 96.15) (width 0.2) (layer "F.Cu") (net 4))
 (via (at 106.5 96.2) (size 0.6) (drill 0.3) (layers "F.Cu" "B.Cu") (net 4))
 (via (at 80 108.3) (size 0.6) (drill 0.3) (layers "F.Cu" "B.Cu") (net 4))
 (segment (start 104.2 98.5) (end 104.2 103.9) (width 0.2) (layer "B.Cu") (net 4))
 (segment (start 82.7 105.6) (end 80 108.3) (width 0.2) (layer "B.Cu") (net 4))
 (segment (start 102.5 105.6) (end 82.7 105.6) (width 0.2) (layer "B.Cu") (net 4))
 (segment (start 106.5 96.2) (end 104.2 98.5) (width 0.2) (layer "B.Cu") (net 4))
 (segment (start 104.2 103.9) (end 102.5 105.6) (width 0.2) (layer "B.Cu") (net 4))
 (segment (start 106.35 86.15) (end 106.3 86.2) (width 0.2) (layer "F.Cu") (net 9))
 (segment (start 80.1 103.3) (end 78.3 103.3) (width 0.2) (layer "F.Cu") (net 9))
 (segment (start 108.25 86.15) (end 106.35 86.15) (width 0.2) (layer "F.Cu") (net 9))
 (via (at 80.1 103.3) (size 0.6) (drill 0.3) (layers "F.Cu" "B.Cu") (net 9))
 (via (at 106.3 86.2) (size 0.6) (drill 0.3) (layers "F.Cu" "B.Cu") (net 9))
 (segment (start 100.6 91.9) (end 100.6 98.1) (width 0.2) (layer "B.Cu") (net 9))
 (segment (start 96.1 102.6) (end 80.8 102.6) (width 0.2) (layer "B.Cu") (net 9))
 (segment (start 100.6 98.1) (end 96.1 102.6) (width 0.2) (layer "B.Cu") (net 9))
 (segment (start 106.3 86.2) (end 100.6 91.9) (width 0.2) (layer "B.Cu") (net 9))
 (segment (start 80.8 102.6) (end 80.1 103.3) (width 0.2) (layer "B.Cu") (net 9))
 (segment (start 97.6 81.5) (end 97.6 83.5) (width 0.2) (layer "F.Cu") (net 15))
 (segment (start 80.1 91.3) (end 78.3 91.3) (width 0.2) (layer "F.Cu") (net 15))
 (via (at 97.6 83.5) (size 0.6) (drill 0.3) (layers "F.Cu" "B.Cu") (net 15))
 (via (at 80.1 91.3) (size 0.6) (drill 0.3) (layers "F.Cu" "B.Cu") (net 15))
 (segment (start 95.6 88.5) (end 92.8 91.3) (width 0.2) (layer "B.Cu") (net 15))
 (segment (start 97.6 83.8) (end 95.6 85.8) (width 0.2) (layer "B.Cu") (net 15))
 (segment (start 97.6 83.5) (end 97.6 83.8) (width 0.2) (layer "B.Cu") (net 15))
 (segment (start 92.8 91.3) (end 80.1 91.3) (width 0.2) (layer "B.Cu") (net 15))
 (segment (start 95.6 85.8) (end 95.6 88.5) (width 0.2) (layer "B.Cu") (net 15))
 (segment (start 106.55 98.15) (end 106.5 98.2) (width 0.2) (layer "F.Cu") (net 3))
 (segment (start 80 109.3) (end 78.3 109.3) (width 0.2) (layer "F.Cu") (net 3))
 (segment (start 108.25 98.15) (end 106.55 98.15) (width 0.2) (layer "F.Cu") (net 3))
 (via (at 80 109.3) (size 0.6) (drill 0.3) (layers "F.Cu" "B.Cu") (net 3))
 (via (at 106.5 98.2) (size 0.6) (drill 0.3) (layers "F.Cu" "B.Cu") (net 3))
 (segment (start 106.5 98.2) (end 104.8 99.9) (width 0.2) (layer "B.Cu") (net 3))
 (segment (start 103.2 106.2) (end 83.1 106.2) (width 0.2) (layer "B.Cu") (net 3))
 (segment (start 83.1 106.2) (end 80 109.3) (width 0.2) (layer "B.Cu") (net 3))
 (segment (start 104.8 104.6) (end 103.2 106.2) (width 0.2) (layer "B.Cu") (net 3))
 (segment (start 104.8 99.9) (end 104.8 104.6) (width 0.2) (layer "B.Cu") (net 3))
 (segment (start 80.1 92.3) (end 78.3 92.3) (width 0.2) (layer "F.Cu") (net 25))
 (segment (start 80.25 92.15) (end 80.1 92.3) (width 0.2) (layer "F.Cu") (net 25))
 (segment (start 84.95 92.15) (end 80.25 92.15) (width 0.2) (layer "F.Cu") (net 25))
 (segment (start 103.6 81.5) (end 103.6 83.5) (width 0.2) (layer "F.Cu") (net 12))
 (segment (start 80.1 97.3) (end 78.3 97.3) (width 0.2) (layer "F.Cu") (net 12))
 (via (at 103.6 83.5) (size 0.6) (drill 0.3) (layers "F.Cu" "B.Cu") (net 12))
 (via (at 80.1 97.3) (size 0.6) (drill 0.3) (layers "F.Cu" "B.Cu") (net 12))
 (segment (start 103.6 83.5) (end 98.1 89) (width 0.2) (layer "B.Cu") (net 12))
 (segment (start 94.4 97.3) (end 80.1 97.3) (width 0.2) (layer "B.Cu") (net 12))
 (segment (start 98.1 89) (end 98.1 93.6) (width 0.2) (layer "B.Cu") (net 12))
 (segment (start 98.1 93.6) (end 94.4 97.3) (width 0.2) (layer "B.Cu") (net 12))
 (segment (start 84.95 86.15) (end 80.25 86.15) (width 0.2) (layer "F.Cu") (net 22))
 (segment (start 80.25 86.15) (end 80.1 86.3) (width 0.2) (layer "F.Cu") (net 22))
 (segment (start 80.1 86.3) (end 78.3 86.3) (width 0.2) (layer "F.Cu") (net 22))
 (segment (start 84.3 96.15) (end 84.15 96.3) (width 0.2) (layer "F.Cu") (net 27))
 (segment (start 84.15 96.3) (end 78.3 96.3) (width 0.2) (layer "F.Cu") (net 27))
 (segment (start 84.95 96.15) (end 84.3 96.15) (width 0.2) (layer "F.Cu") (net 27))
 (segment (start 80.1 93.3) (end 78.3 93.3) (width 0.2) (layer "F.Cu") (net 14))
 (segment (start 99.6 81.5) (end 99.6 83.5) (width 0.2) (layer "F.Cu") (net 14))
 (via (at 80.1 93.3) (size 0.6) (drill 0.3) (layers "F.Cu" "B.Cu") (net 14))
 (via (at 99.6 83.5) (size 0.6) (drill 0.3) (layers "F.Cu" "B.Cu") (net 14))
 (segment (start 96.5 86.6) (end 96.5 90.4) (width 0.2) (layer "B.Cu") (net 14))
 (segment (start 96.5 90.4) (end 93.6 93.3) (width 0.2) (layer "B.Cu") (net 14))
 (segment (start 99.6 83.5) (end 96.5 86.6) (width 0.2) (layer "B.Cu") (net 14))
 (segment (start 93.6 93.3) (end 80.1 93.3) (width 0.2) (layer "B.Cu") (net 14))
 (segment (start 80.25 90.15) (end 80.1 90.3) (width 0.2) (layer "F.Cu") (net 24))
 (segment (start 84.95 90.15) (end 80.25 90.15) (width 0.2) (layer "F.Cu") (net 24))
 (segment (start 80.1 90.3) (end 78.3 90.3) (width 0.2) (layer "F.Cu") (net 24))
 (segment (start 86.1 119.9) (end 87.15 119.9) (width 0.2) (layer "F.Cu") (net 1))
 (segment (start 106.35 102.15) (end 106.3 102.1) (width 0.2) (layer "F.Cu") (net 1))
 (segment (start 87.15 119.9) (end 87.75 120.5) (width 0.2) (layer "F.Cu") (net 1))
 (segment (start 78.3 111.3) (end 80.7 111.3) (width 0.2) (layer "F.Cu") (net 1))
 (segment (start 108.25 102.15) (end 106.35 102.15) (width 0.2) (layer "F.Cu") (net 1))
 (via (at 86.1 119.9) (size 0.6) (drill 0.3) (layers "F.Cu" "B.Cu") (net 1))
 (via (at 106.3 102.1) (size 0.6) (drill 0.3) (layers "F.Cu" "B.Cu") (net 1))
 (via (at 80.7 111.3) (size 0.6) (drill 0.3) (layers "F.Cu" "B.Cu") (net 1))
 (segment (start 106.8 102.6) (end 106.8 118.1) (width 0.2) (layer "B.Cu") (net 1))
 (segment (start 80.7 114.1) (end 84.7 118.1) (width 0.2) (layer "B.Cu") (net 1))
 (segment (start 106.3 102.1) (end 106.8 102.6) (width 0.2) (layer "B.Cu") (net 1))
 (segment (start 80.7 111.3) (end 80.7 114.1) (width 0.2) (layer "B.Cu") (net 1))
 (segment (start 86.1 119.5) (end 86.1 119.9) (width 0.2) (layer "B.Cu") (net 1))
 (segment (start 84.7 118.1) (end 86.1 118.1) (width 0.2) (layer "B.Cu") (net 1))
 (segment (start 106.8 118.1) (end 86.1 118.1) (width 0.2) (layer "B.Cu") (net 1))
 (segment (start 84.7 118.1) (end 86.1 119.5) (width 0.2) (layer "B.Cu") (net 1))
 (segment (start 80.1 88.3) (end 78.3 88.3) (width 0.2) (layer "F.Cu") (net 23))
 (segment (start 84.95 88.15) (end 80.25 88.15) (width 0.2) (layer "F.Cu") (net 23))
 (segment (start 80.25 88.15) (end 80.1 88.3) (width 0.2) (layer "F.Cu") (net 23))
 (segment (start 108.25 90.15) (end 106.35 90.15) (width 0.2) (layer "F.Cu") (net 7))
 (segment (start 80.1 105.3) (end 78.3 105.3) (width 0.2) (layer "F.Cu") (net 7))
 (segment (start 106.35 90.15) (end 106.3 90.2) (width 0.2) (layer "F.Cu") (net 7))
 (via (at 106.3 90.2) (size 0.6) (drill 0.3) (layers "F.Cu" "B.Cu") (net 7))
 (via (at 80.1 105.3) (size 0.6) (drill 0.3) (layers "F.Cu" "B.Cu") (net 7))
 (segment (start 102.2 94.3) (end 102.2 100.5) (width 0.2) (layer "B.Cu") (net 7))
 (segment (start 106.3 90.2) (end 102.2 94.3) (width 0.2) (layer "B.Cu") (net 7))
 (segment (start 98.9 103.8) (end 81.6 103.8) (width 0.2) (layer "B.Cu") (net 7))
 (segment (start 81.6 103.8) (end 80.1 105.3) (width 0.2) (layer "B.Cu") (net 7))
 (segment (start 102.2 100.5) (end 98.9 103.8) (width 0.2) (layer "B.Cu") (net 7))
 (segment (start 105.6 81.5) (end 105.6 83.4) (width 0.2) (layer "F.Cu") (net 11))
 (segment (start 80.1 99.3) (end 78.3 99.3) (width 0.2) (layer "F.Cu") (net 11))
 (via (at 80.1 99.3) (size 0.6) (drill 0.3) (layers "F.Cu" "B.Cu") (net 11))
 (via (at 105.6 83.4) (size 0.6) (drill 0.3) (layers "F.Cu" "B.Cu") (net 11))
 (segment (start 95.1 99.3) (end 80.1 99.3) (width 0.2) (layer "B.Cu") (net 11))
 (segment (start 98.9 95.5) (end 95.1 99.3) (width 0.2) (layer "B.Cu") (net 11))
 (segment (start 105.6 83.4) (end 105.6 83.5) (width 0.2) (layer "B.Cu") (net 11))
 (segment (start 105.6 83.5) (end 98.9 90.2) (width 0.2) (layer "B.Cu") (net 11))
 (segment (start 98.9 90.2) (end 98.9 95.5) (width 0.2) (layer "B.Cu") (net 11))
 (segment (start 80.1 102.3) (end 78.3 102.3) (width 0.2) (layer "F.Cu") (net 30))
 (segment (start 84.95 102.15) (end 80.25 102.15) (width 0.2) (layer "F.Cu") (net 30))
 (segment (start 80.25 102.15) (end 80.1 102.3) (width 0.2) (layer "F.Cu") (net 30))
 (segment (start 108.25 84.15) (end 106.35 84.15) (width 0.2) (layer "F.Cu") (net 10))
 (segment (start 80.1 101.3) (end 78.3 101.3) (width 0.2) (layer "F.Cu") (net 10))
 (segment (start 106.35 84.15) (end 106.3 84.2) (width 0.2) (layer "F.Cu") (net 10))
 (via (at 80.1 101.3) (size 0.6) (drill 0.3) (layers "F.Cu" "B.Cu") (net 10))
 (via (at 106.3 84.2) (size 0.6) (drill 0.3) (layers "F.Cu" "B.Cu") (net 10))
 (segment (start 106.3 84.2) (end 99.8 90.7) (width 0.2) (layer "B.Cu") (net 10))
 (segment (start 99.8 90.7) (end 99.8 96.6) (width 0.2) (layer "B.Cu") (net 10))
 (segment (start 99.8 96.6) (end 95.1 101.3) (width 0.2) (layer "B.Cu") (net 10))
 (segment (start 95.1 101.3) (end 80.1 101.3) (width 0.2) (layer "B.Cu") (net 10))
 (segment (start 106.35 92.15) (end 106.3 92.2) (width 0.2) (layer "F.Cu") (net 6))
 (segment (start 108.25 92.15) (end 106.35 92.15) (width 0.2) (layer "F.Cu") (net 6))
 (segment (start 80.1 106.3) (end 78.3 106.3) (width 0.2) (layer "F.Cu") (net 6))
 (via (at 80.1 106.3) (size 0.6) (drill 0.3) (layers "F.Cu" "B.Cu") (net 6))
 (via (at 106.3 92.2) (size 0.6) (drill 0.3) (layers "F.Cu" "B.Cu") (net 6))
 (segment (start 100 104.4) (end 82 104.4) (width 0.2) (layer "B.Cu") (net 6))
 (segment (start 82 104.4) (end 80.1 106.3) (width 0.2) (layer "B.Cu") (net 6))
 (segment (start 102.9 95.6) (end 102.9 101.5) (width 0.2) (layer "B.Cu") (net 6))
 (segment (start 102.9 101.5) (end 100 104.4) (width 0.2) (layer "B.Cu") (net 6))
 (segment (start 106.3 92.2) (end 102.9 95.6) (width 0.2) (layer "B.Cu") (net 6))
 (segment (start 106.55 100.15) (end 106.5 100.2) (width 0.2) (layer "F.Cu") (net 2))
 (segment (start 80 110.3) (end 78.3 110.3) (width 0.2) (layer "F.Cu") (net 2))
 (segment (start 108.25 100.15) (end 106.55 100.15) (width 0.2) (layer "F.Cu") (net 2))
 (via (at 106.5 100.2) (size 0.6) (drill 0.3) (layers "F.Cu" "B.Cu") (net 2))
 (via (at 80 110.3) (size 0.6) (drill 0.3) (layers "F.Cu" "B.Cu") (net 2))
 (segment (start 80 110.3) (end 83.3 107) (width 0.2) (layer "B.Cu") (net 2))
 (segment (start 83.3 107) (end 103.5 107) (width 0.2) (layer "B.Cu") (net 2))
 (segment (start 103.5 107) (end 105.6 104.9) (width 0.2) (layer "B.Cu") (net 2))
 (segment (start 105.6 104.9) (end 105.6 101.1) (width 0.2) (layer "B.Cu") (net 2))
 (segment (start 105.6 101.1) (end 106.5 100.2) (width 0.2) (layer "B.Cu") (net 2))
 (segment (start 80.1 89.3) (end 78.3 89.3) (width 0.2) (layer "F.Cu") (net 16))
 (segment (start 95.6 81.5) (end 95.6 83.5) (width 0.2) (layer "F.Cu") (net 16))
 (via (at 80.1 89.3) (size 0.6) (drill 0.3) (layers "F.Cu" "B.Cu") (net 16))
 (via (at 95.6 83.5) (size 0.6) (drill 0.3) (layers "F.Cu" "B.Cu") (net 16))
 (segment (start 94.7 85.3) (end 94.7 87.4) (width 0.2) (layer "B.Cu") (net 16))
 (segment (start 94.7 87.4) (end 92.8 89.3) (width 0.2) (layer "B.Cu") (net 16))
 (segment (start 92.8 89.3) (end 80.1 89.3) (width 0.2) (layer "B.Cu") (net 16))
 (segment (start 95.6 84.4) (end 94.7 85.3) (width 0.2) (layer "B.Cu") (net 16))
 (segment (start 95.6 83.5) (end 95.6 84.4) (width 0.2) (layer "B.Cu") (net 16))
 (segment (start 80.1 95.3) (end 78.3 95.3) (width 0.2) (layer "F.Cu") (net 13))
 (segment (start 101.6 81.5) (end 101.6 83.5) (width 0.2) (layer "F.Cu") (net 13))
 (via (at 80.1 95.3) (size 0.6) (drill 0.3) (layers "F.Cu" "B.Cu") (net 13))
 (via (at 101.6 83.5) (size 0.6) (drill 0.3) (layers "F.Cu" "B.Cu") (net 13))
 (segment (start 101.6 83.5) (end 97.3 87.8) (width 0.2) (layer "B.Cu") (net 13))
 (segment (start 97.3 87.8) (end 97.3 92.3) (width 0.2) (layer "B.Cu") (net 13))
 (segment (start 94.3 95.3) (end 80.1 95.3) (width 0.2) (layer "B.Cu") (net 13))
 (segment (start 97.3 92.3) (end 94.3 95.3) (width 0.2) (layer "B.Cu") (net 13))
 (segment (start 89.6 76.5) (end 89.5 76.4) (width 0.2) (layer "F.Cu") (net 19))
 (segment (start 89.6 81.5) (end 89.6 76.5) (width 0.2) (layer "F.Cu") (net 19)))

